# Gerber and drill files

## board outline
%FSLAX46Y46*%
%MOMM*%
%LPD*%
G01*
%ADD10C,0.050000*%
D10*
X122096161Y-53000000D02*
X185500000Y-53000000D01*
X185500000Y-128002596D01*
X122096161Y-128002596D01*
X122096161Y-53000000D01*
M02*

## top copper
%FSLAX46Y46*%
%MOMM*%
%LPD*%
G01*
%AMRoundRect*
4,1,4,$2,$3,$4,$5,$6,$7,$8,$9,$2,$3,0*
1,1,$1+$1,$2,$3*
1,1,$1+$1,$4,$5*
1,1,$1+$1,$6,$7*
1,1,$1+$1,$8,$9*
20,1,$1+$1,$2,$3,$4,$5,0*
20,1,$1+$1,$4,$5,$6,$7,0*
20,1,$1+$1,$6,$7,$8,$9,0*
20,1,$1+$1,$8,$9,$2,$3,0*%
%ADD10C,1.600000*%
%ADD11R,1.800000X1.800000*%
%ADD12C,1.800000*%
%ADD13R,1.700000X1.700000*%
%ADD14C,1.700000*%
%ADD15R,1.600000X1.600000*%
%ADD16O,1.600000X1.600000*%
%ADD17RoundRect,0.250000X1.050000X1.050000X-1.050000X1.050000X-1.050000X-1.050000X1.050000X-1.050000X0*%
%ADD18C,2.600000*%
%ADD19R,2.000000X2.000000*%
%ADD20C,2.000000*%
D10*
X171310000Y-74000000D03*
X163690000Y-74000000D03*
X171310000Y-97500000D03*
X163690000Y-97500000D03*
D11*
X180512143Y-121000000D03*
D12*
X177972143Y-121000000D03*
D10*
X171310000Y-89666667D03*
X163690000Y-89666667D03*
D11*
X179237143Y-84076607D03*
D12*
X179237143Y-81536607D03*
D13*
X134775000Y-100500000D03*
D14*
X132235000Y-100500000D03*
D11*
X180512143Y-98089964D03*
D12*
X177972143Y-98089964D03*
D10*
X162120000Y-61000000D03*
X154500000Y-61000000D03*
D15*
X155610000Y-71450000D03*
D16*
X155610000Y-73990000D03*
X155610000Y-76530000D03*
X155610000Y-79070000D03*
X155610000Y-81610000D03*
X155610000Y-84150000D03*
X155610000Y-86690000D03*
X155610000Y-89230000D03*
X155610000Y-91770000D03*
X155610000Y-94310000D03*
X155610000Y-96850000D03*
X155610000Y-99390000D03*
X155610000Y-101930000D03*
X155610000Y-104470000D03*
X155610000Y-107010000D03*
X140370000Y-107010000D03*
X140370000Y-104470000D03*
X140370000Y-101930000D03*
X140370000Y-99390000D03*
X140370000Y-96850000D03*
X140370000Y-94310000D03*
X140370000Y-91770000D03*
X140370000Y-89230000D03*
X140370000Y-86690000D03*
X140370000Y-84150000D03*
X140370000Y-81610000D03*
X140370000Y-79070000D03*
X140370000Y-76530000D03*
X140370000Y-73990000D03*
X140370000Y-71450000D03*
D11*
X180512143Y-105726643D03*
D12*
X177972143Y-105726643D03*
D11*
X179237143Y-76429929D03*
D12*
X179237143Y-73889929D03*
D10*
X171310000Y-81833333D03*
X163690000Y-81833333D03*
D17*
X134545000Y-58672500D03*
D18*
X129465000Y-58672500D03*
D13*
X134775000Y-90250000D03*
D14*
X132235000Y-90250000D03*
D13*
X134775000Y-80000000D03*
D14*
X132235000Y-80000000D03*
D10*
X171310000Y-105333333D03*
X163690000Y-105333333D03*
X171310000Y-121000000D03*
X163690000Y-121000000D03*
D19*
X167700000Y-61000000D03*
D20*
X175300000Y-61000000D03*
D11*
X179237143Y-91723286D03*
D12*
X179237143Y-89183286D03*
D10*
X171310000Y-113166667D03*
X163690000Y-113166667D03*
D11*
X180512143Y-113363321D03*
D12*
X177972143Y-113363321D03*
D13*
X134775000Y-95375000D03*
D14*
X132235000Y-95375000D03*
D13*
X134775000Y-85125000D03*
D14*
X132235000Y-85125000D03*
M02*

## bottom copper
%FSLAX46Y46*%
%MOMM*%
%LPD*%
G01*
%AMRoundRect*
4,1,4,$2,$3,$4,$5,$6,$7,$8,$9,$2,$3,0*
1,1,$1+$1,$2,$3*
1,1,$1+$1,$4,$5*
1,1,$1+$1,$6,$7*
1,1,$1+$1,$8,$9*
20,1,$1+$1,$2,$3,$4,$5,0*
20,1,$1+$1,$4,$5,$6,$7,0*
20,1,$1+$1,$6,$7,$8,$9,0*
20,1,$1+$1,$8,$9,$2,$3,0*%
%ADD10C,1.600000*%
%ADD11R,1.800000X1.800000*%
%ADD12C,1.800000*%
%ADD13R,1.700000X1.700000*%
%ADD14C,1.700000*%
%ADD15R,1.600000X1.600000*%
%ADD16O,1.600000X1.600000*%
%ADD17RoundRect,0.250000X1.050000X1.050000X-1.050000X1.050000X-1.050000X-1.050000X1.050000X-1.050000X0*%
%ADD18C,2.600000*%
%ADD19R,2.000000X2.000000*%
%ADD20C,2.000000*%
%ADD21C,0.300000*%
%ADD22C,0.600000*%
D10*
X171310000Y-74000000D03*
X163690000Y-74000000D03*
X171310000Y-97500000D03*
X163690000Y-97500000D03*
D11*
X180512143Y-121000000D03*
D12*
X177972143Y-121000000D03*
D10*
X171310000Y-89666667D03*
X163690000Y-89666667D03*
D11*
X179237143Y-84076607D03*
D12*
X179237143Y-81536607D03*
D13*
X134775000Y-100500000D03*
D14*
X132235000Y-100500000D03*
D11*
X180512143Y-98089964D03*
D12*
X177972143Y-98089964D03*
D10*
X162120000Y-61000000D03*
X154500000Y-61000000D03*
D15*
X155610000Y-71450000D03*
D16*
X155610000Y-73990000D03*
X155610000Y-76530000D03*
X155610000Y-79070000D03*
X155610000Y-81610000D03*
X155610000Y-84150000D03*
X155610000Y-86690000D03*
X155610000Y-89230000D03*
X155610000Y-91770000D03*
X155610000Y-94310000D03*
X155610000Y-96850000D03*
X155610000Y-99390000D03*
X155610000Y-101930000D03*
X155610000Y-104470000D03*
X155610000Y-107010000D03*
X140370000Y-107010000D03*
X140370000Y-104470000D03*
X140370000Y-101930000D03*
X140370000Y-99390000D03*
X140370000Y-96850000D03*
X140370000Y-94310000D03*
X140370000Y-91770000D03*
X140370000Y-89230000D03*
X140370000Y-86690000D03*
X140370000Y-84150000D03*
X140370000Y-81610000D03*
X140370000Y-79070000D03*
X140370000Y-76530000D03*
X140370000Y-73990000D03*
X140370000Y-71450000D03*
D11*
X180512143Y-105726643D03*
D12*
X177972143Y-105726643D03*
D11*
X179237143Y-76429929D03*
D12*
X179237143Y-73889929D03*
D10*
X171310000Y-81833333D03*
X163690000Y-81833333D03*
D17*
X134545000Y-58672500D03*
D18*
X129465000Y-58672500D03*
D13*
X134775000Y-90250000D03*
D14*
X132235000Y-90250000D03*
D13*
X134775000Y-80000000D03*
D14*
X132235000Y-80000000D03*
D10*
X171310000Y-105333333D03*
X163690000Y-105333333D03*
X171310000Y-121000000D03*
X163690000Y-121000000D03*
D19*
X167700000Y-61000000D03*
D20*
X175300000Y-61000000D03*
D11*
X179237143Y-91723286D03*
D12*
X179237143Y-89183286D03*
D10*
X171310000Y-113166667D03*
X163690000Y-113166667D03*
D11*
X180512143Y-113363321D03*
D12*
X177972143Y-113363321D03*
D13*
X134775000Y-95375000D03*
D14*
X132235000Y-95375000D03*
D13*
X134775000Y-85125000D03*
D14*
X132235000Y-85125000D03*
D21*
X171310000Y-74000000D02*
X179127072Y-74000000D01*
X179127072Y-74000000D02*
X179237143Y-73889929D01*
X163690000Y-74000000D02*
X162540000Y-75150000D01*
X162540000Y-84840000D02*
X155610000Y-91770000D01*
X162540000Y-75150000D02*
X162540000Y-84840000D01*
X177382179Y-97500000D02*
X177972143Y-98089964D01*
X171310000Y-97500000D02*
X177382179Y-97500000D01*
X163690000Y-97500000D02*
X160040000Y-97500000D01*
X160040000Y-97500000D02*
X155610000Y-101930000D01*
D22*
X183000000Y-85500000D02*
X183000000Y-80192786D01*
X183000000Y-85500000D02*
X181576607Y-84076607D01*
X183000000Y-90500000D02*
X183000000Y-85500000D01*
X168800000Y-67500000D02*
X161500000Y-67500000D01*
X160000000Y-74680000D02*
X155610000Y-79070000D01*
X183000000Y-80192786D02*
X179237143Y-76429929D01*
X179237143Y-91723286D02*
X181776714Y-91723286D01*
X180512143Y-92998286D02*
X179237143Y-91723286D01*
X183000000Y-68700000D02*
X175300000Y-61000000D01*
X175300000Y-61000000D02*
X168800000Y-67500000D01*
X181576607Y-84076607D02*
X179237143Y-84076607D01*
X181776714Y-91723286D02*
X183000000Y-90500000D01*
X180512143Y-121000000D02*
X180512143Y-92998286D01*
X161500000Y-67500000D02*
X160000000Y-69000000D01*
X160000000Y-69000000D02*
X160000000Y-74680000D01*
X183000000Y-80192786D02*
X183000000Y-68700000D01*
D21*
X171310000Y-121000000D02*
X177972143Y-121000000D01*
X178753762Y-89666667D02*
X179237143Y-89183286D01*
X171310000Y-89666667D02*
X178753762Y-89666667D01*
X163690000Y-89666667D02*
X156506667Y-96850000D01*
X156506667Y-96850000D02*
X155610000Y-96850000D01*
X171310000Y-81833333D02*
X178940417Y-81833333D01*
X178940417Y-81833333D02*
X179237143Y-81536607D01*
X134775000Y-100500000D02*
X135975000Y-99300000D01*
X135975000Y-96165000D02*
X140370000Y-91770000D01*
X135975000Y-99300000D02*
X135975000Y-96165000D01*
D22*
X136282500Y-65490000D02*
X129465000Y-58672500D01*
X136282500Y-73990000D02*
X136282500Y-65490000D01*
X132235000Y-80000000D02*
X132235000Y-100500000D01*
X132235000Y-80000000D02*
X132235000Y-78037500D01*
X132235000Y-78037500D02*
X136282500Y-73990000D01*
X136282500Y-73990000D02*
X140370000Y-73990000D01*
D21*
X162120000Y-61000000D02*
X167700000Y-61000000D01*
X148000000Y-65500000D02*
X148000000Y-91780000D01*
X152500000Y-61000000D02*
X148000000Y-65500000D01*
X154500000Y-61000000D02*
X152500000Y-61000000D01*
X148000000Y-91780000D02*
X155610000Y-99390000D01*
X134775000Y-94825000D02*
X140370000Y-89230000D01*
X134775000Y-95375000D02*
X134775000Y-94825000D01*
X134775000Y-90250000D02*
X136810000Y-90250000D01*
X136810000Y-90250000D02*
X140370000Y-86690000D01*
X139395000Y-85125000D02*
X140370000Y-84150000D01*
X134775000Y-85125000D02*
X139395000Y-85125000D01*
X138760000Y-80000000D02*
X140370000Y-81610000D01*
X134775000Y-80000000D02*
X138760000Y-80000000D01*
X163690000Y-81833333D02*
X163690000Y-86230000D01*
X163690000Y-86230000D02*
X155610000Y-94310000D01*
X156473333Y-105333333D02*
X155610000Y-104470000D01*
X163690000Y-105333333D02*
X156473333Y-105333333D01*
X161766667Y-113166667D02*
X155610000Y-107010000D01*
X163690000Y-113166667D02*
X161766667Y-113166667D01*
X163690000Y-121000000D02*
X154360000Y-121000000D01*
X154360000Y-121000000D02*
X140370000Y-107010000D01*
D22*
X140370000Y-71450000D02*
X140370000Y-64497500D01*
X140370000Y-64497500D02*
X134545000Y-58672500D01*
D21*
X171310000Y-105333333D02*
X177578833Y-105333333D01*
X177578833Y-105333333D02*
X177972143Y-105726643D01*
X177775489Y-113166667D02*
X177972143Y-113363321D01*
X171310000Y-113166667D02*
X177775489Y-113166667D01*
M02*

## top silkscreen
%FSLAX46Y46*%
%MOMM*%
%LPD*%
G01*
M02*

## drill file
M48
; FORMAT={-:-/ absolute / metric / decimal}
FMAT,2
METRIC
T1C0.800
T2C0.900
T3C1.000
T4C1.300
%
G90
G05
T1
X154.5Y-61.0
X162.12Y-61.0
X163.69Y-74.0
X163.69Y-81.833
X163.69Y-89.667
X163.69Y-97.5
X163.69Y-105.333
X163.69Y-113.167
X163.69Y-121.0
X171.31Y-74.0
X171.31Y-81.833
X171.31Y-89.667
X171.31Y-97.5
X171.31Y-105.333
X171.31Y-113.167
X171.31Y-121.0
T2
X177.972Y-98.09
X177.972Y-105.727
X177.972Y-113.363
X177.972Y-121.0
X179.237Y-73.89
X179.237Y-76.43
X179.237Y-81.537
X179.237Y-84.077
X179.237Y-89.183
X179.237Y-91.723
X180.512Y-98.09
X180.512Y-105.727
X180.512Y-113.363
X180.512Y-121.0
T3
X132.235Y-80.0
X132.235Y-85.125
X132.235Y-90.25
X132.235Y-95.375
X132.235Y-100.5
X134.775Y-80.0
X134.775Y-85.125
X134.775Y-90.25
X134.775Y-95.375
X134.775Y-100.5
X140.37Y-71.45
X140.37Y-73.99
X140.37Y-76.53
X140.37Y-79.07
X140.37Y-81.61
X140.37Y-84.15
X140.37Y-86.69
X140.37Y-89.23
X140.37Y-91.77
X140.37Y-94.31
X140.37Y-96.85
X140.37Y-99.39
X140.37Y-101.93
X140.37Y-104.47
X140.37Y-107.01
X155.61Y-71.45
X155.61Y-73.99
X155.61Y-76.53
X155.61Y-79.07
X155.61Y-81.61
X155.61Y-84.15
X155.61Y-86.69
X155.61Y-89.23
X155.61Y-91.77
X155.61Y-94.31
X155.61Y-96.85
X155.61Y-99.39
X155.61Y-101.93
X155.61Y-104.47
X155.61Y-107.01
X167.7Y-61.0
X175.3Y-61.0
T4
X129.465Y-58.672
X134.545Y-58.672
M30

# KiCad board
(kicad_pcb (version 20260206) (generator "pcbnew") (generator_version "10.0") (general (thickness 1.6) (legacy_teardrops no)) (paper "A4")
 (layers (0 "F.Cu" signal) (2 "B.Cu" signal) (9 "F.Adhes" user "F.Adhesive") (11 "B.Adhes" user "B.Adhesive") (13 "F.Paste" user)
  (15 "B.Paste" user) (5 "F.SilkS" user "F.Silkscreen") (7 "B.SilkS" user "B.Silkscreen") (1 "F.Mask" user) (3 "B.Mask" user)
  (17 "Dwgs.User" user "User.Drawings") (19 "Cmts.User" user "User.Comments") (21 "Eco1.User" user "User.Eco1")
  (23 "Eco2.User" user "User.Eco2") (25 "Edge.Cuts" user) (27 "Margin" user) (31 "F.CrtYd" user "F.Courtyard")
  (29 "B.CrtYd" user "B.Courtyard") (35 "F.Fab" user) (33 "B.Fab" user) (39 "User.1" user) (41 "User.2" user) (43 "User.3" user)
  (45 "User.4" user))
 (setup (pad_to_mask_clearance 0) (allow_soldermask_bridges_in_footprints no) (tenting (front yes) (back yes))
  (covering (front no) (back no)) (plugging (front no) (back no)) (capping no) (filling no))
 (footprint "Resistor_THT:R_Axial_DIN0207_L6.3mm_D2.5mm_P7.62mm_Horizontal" (layer "B.Cu") (at 171.31 74 180)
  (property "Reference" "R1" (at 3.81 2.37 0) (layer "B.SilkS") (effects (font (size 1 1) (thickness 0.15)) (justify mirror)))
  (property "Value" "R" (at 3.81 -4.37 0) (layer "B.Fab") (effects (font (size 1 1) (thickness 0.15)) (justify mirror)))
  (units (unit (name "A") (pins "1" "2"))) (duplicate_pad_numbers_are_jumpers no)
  (pad "1" thru_hole circle (at 0 0 180) (size 1.6 1.6) (drill 0.8) (layers "*.Cu" "*.Mask") (remove_unused_layers no)
   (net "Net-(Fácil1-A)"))
  (pad "2" thru_hole circle (at 7.62 0 180) (size 1.6 1.6) (drill 0.8) (layers "*.Cu" "*.Mask") (remove_unused_layers no)
   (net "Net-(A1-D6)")))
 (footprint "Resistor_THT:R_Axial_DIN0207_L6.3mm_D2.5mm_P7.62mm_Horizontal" (layer "B.Cu") (at 171.31 97.5 180)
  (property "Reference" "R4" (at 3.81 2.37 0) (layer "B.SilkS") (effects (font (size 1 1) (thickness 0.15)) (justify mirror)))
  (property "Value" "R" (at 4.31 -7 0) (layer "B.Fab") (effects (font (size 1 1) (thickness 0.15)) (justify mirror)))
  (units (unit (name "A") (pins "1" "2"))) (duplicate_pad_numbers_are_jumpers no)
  (pad "1" thru_hole circle (at 0 0 180) (size 1.6 1.6) (drill 0.8) (layers "*.Cu" "*.Mask") (remove_unused_layers no)
   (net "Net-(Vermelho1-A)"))
  (pad "2" thru_hole circle (at 7.62 0 180) (size 1.6 1.6) (drill 0.8) (layers "*.Cu" "*.Mask") (remove_unused_layers no)
   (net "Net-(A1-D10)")))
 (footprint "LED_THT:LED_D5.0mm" (layer "B.Cu") (at 180.512143 121 180)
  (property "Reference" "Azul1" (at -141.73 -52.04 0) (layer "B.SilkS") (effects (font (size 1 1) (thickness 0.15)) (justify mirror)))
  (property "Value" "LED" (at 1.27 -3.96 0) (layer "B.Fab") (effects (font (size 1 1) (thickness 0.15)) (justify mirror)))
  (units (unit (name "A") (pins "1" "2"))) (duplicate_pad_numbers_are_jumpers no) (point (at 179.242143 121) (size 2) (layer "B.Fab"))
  (pad "1" thru_hole rect (at 0 0 180) (size 1.8 1.8) (drill 0.9) (layers "*.Cu" "*.Mask") (remove_unused_layers no)
   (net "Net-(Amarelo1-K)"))
  (pad "2" thru_hole circle (at 2.54 0 180) (size 1.8 1.8) (drill 0.9) (layers "*.Cu" "*.Mask") (remove_unused_layers no)
   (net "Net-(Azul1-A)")))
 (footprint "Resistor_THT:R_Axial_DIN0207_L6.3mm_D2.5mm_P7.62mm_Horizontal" (layer "B.Cu") (at 171.31 89.666667 180)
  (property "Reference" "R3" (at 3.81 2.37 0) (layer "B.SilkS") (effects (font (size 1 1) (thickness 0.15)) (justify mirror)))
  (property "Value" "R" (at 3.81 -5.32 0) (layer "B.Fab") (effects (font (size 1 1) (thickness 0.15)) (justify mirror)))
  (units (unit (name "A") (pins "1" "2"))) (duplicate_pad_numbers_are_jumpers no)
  (pad "1" thru_hole circle (at 0 0 180) (size 1.6 1.6) (drill 0.8) (layers "*.Cu" "*.Mask") (remove_unused_layers no)
   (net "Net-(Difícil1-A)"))
  (pad "2" thru_hole circle (at 7.62 0 180) (size 1.6 1.6) (drill 0.8) (layers "*.Cu" "*.Mask") (remove_unused_layers no)
   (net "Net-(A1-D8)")))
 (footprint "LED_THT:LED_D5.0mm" (layer "B.Cu") (at 179.237143 84.076607 90)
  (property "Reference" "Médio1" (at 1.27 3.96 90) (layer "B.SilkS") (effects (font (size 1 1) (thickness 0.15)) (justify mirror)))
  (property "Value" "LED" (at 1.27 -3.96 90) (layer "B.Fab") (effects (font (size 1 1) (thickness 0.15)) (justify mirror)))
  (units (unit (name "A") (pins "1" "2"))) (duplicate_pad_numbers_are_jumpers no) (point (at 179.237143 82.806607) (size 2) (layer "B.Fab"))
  (pad "1" thru_hole rect (at 0 0 90) (size 1.8 1.8) (drill 0.9) (layers "*.Cu" "*.Mask") (remove_unused_layers no) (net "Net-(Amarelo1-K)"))
  (pad "2" thru_hole circle (at 2.54 0 90) (size 1.8 1.8) (drill 0.9) (layers "*.Cu" "*.Mask") (remove_unused_layers no)
   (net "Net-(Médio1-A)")))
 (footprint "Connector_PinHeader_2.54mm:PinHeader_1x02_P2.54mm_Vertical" (layer "B.Cu") (at 134.775 100.5 90)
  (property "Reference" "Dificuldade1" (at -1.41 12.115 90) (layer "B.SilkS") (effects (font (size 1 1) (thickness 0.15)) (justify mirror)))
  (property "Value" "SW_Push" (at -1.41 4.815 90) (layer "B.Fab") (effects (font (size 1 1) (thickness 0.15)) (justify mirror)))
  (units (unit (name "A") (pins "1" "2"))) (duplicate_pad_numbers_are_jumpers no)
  (pad "1" thru_hole rect (at 0 0 90) (size 1.7 1.7) (drill 1) (layers "*.Cu" "*.Mask") (remove_unused_layers no) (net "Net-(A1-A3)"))
  (pad "2" thru_hole circle (at 0 -2.54 90) (size 1.7 1.7) (drill 1) (layers "*.Cu" "*.Mask") (remove_unused_layers no)
   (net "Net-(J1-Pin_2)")))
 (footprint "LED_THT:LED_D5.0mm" (layer "B.Cu") (at 180.512143 98.089964 180)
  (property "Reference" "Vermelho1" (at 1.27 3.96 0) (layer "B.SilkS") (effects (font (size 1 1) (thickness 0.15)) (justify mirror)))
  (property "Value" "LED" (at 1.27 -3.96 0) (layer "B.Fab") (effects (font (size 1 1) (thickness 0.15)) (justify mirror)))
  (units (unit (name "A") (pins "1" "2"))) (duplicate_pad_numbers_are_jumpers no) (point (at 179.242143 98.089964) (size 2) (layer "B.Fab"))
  (pad "1" thru_hole rect (at 0 0 180) (size 1.8 1.8) (drill 0.9) (layers "*.Cu" "*.Mask") (remove_unused_layers no)
   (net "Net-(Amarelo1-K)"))
  (pad "2" thru_hole circle (at 2.54 0 180) (size 1.8 1.8) (drill 0.9) (layers "*.Cu" "*.Mask") (remove_unused_layers no)
   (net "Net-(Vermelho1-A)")))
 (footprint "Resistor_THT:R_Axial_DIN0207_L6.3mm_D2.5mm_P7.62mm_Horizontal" (layer "B.Cu") (at 162.12 61 180)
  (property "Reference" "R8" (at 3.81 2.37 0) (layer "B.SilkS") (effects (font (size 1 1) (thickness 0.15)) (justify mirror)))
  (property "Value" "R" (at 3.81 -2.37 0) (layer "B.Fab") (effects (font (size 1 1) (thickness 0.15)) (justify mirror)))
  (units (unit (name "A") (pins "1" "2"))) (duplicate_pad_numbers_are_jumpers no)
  (pad "1" thru_hole circle (at 0 0 180) (size 1.6 1.6) (drill 0.8) (layers "*.Cu" "*.Mask") (remove_unused_layers no) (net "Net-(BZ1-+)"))
  (pad "2" thru_hole circle (at 7.62 0 180) (size 1.6 1.6) (drill 0.8) (layers "*.Cu" "*.Mask") (remove_unused_layers no)
   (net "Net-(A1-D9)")))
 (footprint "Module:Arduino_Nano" (layer "B.Cu") (at 155.61 71.45 180)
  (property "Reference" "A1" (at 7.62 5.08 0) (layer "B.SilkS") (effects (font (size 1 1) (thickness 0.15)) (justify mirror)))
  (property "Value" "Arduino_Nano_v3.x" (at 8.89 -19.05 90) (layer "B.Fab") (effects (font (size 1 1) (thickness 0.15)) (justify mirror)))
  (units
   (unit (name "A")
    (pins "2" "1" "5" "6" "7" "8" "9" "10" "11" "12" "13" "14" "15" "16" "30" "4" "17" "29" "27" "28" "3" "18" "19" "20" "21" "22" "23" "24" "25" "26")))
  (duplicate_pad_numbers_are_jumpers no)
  (pad "1" thru_hole rect (at 0 0 180) (size 1.6 1.6) (drill 1) (layers "*.Cu" "*.Mask") (remove_unused_layers no)
   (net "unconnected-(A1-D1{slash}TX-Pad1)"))
  (pad "2" thru_hole oval (at 0 -2.54 180) (size 1.6 1.6) (drill 1) (layers "*.Cu" "*.Mask") (remove_unused_layers no)
   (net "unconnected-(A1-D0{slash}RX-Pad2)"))
  (pad "3" thru_hole oval (at 0 -5.08 180) (size 1.6 1.6) (drill 1) (layers "*.Cu" "*.Mask") (remove_unused_layers no)
   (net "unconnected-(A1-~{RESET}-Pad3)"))
  (pad "4" thru_hole oval (at 0 -7.62 180) (size 1.6 1.6) (drill 1) (layers "*.Cu" "*.Mask") (remove_unused_layers no)
   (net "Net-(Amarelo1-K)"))
  (pad "5" thru_hole oval (at 0 -10.16 180) (size 1.6 1.6) (drill 1) (layers "*.Cu" "*.Mask") (remove_unused_layers no) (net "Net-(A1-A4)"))
  (pad "6" thru_hole oval (at 0 -12.7 180) (size 1.6 1.6) (drill 1) (layers "*.Cu" "*.Mask") (remove_unused_layers no) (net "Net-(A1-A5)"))
  (pad "7" thru_hole oval (at 0 -15.24 180) (size 1.6 1.6) (drill 1) (layers "*.Cu" "*.Mask") (remove_unused_layers no) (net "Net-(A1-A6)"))
  (pad "8" thru_hole oval (at 0 -17.78 180) (size 1.6 1.6) (drill 1) (layers "*.Cu" "*.Mask") (remove_unused_layers no) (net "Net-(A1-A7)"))
  (pad "9" thru_hole oval (at 0 -20.32 180) (size 1.6 1.6) (drill 1) (layers "*.Cu" "*.Mask") (remove_unused_layers no) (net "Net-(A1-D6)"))
  (pad "10" thru_hole oval (at 0 -22.86 180) (size 1.6 1.6) (drill 1) (layers "*.Cu" "*.Mask") (remove_unused_layers no) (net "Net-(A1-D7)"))
  (pad "11" thru_hole oval (at 0 -25.4 180) (size 1.6 1.6) (drill 1) (layers "*.Cu" "*.Mask") (remove_unused_layers no) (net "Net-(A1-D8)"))
  (pad "12" thru_hole oval (at 0 -27.94 180) (size 1.6 1.6) (drill 1) (layers "*.Cu" "*.Mask") (remove_unused_layers no) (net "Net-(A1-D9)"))
  (pad "13" thru_hole oval (at 0 -30.48 180) (size 1.6 1.6) (drill 1) (layers "*.Cu" "*.Mask") (remove_unused_layers no)
   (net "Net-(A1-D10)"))
  (pad "14" thru_hole oval (at 0 -33.02 180) (size 1.6 1.6) (drill 1) (layers "*.Cu" "*.Mask") (remove_unused_layers no)
   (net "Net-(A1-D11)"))
  (pad "15" thru_hole oval (at 0 -35.56 180) (size 1.6 1.6) (drill 1) (layers "*.Cu" "*.Mask") (remove_unused_layers no)
   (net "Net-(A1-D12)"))
  (pad "16" thru_hole oval (at 15.24 -35.56 180) (size 1.6 1.6) (drill 1) (layers "*.Cu" "*.Mask") (remove_unused_layers no)
   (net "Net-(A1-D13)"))
  (pad "17" thru_hole oval (at 15.24 -33.02 180) (size 1.6 1.6) (drill 1) (layers "*.Cu" "*.Mask") (remove_unused_layers no)
   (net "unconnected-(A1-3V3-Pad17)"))
  (pad "18" thru_hole oval (at 15.24 -30.48 180) (size 1.6 1.6) (drill 1) (layers "*.Cu" "*.Mask") (remove_unused_layers no)
   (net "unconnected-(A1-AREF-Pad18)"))
  (pad "19" thru_hole oval (at 15.24 -27.94 180) (size 1.6 1.6) (drill 1) (layers "*.Cu" "*.Mask") (remove_unused_layers no)
   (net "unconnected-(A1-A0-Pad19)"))
  (pad "20" thru_hole oval (at 15.24 -25.4 180) (size 1.6 1.6) (drill 1) (layers "*.Cu" "*.Mask") (remove_unused_layers no)
   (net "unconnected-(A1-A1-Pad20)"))
  (pad "21" thru_hole oval (at 15.24 -22.86 180) (size 1.6 1.6) (drill 1) (layers "*.Cu" "*.Mask") (remove_unused_layers no)
   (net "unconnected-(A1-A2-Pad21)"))
  (pad "22" thru_hole oval (at 15.24 -20.32 180) (size 1.6 1.6) (drill 1) (layers "*.Cu" "*.Mask") (remove_unused_layers no)
   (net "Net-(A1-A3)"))
  (pad "23" thru_hole oval (at 15.24 -17.78 180) (size 1.6 1.6) (drill 1) (layers "*.Cu" "*.Mask") (remove_unused_layers no)
   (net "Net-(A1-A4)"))
  (pad "24" thru_hole oval (at 15.24 -15.24 180) (size 1.6 1.6) (drill 1) (layers "*.Cu" "*.Mask") (remove_unused_layers no)
   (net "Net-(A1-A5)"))
  (pad "25" thru_hole oval (at 15.24 -12.7 180) (size 1.6 1.6) (drill 1) (layers "*.Cu" "*.Mask") (remove_unused_layers no)
   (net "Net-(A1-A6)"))
  (pad "26" thru_hole oval (at 15.24 -10.16 180) (size 1.6 1.6) (drill 1) (layers "*.Cu" "*.Mask") (remove_unused_layers no)
   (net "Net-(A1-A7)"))
  (pad "27" thru_hole oval (at 15.24 -7.62 180) (size 1.6 1.6) (drill 1) (layers "*.Cu" "*.Mask") (remove_unused_layers no)
   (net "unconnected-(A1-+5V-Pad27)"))
  (pad "28" thru_hole oval (at 15.24 -5.08 180) (size 1.6 1.6) (drill 1) (layers "*.Cu" "*.Mask") (remove_unused_layers no)
   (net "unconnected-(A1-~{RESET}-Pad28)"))
  (pad "29" thru_hole oval (at 15.24 -2.54 180) (size 1.6 1.6) (drill 1) (layers "*.Cu" "*.Mask") (remove_unused_layers no)
   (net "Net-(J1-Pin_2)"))
  (pad "30" thru_hole oval (at 15.24 0 180) (size 1.6 1.6) (drill 1) (layers "*.Cu" "*.Mask") (remove_unused_layers no) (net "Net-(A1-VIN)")))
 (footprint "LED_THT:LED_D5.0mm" (layer "B.Cu") (at 180.512143 105.726643 180)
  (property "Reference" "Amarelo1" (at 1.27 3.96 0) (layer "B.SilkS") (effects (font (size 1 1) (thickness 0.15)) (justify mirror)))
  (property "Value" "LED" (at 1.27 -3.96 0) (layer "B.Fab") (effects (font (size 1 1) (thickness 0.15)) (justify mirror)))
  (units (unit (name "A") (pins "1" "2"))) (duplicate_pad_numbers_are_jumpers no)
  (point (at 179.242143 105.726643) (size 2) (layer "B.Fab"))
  (pad "1" thru_hole rect (at 0 0 180) (size 1.8 1.8) (drill 0.9) (layers "*.Cu" "*.Mask") (remove_unused_layers no)
   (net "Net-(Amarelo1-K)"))
  (pad "2" thru_hole circle (at 2.54 0 180) (size 1.8 1.8) (drill 0.9) (layers "*.Cu" "*.Mask") (remove_unused_layers no)
   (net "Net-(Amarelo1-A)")))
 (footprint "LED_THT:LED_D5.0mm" (layer "B.Cu") (at 179.237143 76.429929 90)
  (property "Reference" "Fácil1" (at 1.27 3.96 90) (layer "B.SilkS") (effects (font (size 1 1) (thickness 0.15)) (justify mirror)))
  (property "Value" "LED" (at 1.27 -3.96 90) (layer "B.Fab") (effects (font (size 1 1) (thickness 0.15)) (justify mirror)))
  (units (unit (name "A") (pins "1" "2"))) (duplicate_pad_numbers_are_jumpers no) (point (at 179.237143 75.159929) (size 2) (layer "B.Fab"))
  (pad "1" thru_hole rect (at 0 0 90) (size 1.8 1.8) (drill 0.9) (layers "*.Cu" "*.Mask") (remove_unused_layers no) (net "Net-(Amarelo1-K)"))
  (pad "2" thru_hole circle (at 2.54 0 90) (size 1.8 1.8) (drill 0.9) (layers "*.Cu" "*.Mask") (remove_unused_layers no)
   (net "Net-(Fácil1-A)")))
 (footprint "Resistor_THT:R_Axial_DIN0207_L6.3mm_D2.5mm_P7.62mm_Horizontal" (layer "B.Cu") (at 171.31 81.833333 180)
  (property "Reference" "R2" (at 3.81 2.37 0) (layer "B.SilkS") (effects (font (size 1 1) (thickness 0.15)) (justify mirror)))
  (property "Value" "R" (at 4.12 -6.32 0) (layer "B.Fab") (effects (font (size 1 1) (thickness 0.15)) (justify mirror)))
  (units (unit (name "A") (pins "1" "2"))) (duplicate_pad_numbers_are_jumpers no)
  (pad "1" thru_hole circle (at 0 0 180) (size 1.6 1.6) (drill 0.8) (layers "*.Cu" "*.Mask") (remove_unused_layers no)
   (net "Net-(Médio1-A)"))
  (pad "2" thru_hole circle (at 7.62 0 180) (size 1.6 1.6) (drill 0.8) (layers "*.Cu" "*.Mask") (remove_unused_layers no)
   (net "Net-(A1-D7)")))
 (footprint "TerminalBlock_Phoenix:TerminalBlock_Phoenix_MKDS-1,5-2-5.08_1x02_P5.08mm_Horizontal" (layer "B.Cu") (at 134.545 58.6725 180)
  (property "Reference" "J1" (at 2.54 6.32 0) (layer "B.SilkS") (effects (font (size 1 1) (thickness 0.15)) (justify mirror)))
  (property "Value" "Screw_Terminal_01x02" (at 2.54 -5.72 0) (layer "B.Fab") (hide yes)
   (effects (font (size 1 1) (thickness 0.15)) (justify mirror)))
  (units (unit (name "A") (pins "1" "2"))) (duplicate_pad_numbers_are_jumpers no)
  (pad "1" thru_hole roundrect (at 0 0 180) (size 2.6 2.6) (drill 1.3) (layers "*.Cu" "*.Mask") (remove_unused_layers no)
   (roundrect_rratio 0.096154) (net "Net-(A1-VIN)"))
  (pad "2" thru_hole circle (at 5.08 0 180) (size 2.6 2.6) (drill 1.3) (layers "*.Cu" "*.Mask") (remove_unused_layers no)
   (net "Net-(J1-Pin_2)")))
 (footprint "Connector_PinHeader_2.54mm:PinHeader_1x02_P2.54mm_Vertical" (layer "B.Cu") (at 134.775 90.25 90)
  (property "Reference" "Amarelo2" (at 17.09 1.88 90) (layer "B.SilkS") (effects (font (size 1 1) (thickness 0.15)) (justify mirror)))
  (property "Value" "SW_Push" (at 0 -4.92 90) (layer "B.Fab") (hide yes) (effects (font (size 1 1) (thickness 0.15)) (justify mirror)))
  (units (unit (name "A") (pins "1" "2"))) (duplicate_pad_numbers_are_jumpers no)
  (pad "1" thru_hole rect (at 0 0 90) (size 1.7 1.7) (drill 1) (layers "*.Cu" "*.Mask") (remove_unused_layers no) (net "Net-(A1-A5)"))
  (pad "2" thru_hole circle (at 0 -2.54 90) (size 1.7 1.7) (drill 1) (layers "*.Cu" "*.Mask") (remove_unused_layers no)
   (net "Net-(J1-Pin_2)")))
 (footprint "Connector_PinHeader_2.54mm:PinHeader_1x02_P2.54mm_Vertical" (layer "B.Cu") (at 134.775 80 90)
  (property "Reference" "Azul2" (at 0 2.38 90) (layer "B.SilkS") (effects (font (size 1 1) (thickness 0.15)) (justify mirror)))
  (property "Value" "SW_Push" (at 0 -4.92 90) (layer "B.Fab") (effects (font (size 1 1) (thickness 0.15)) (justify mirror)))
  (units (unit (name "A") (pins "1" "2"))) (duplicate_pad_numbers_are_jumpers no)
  (pad "1" thru_hole rect (at 0 0 90) (size 1.7 1.7) (drill 1) (layers "*.Cu" "*.Mask") (remove_unused_layers no) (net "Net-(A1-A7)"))
  (pad "2" thru_hole circle (at 0 -2.54 90) (size 1.7 1.7) (drill 1) (layers "*.Cu" "*.Mask") (remove_unused_layers no)
   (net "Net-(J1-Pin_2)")))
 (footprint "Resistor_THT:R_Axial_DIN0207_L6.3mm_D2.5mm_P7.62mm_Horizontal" (layer "B.Cu") (at 171.31 105.333333 180)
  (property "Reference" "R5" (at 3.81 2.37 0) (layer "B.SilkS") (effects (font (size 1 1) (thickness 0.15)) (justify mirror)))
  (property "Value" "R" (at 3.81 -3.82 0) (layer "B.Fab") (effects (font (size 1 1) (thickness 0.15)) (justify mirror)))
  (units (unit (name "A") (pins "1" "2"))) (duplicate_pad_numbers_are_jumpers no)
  (pad "1" thru_hole circle (at 0 0 180) (size 1.6 1.6) (drill 0.8) (layers "*.Cu" "*.Mask") (remove_unused_layers no)
   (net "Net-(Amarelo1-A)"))
  (pad "2" thru_hole circle (at 7.62 0 180) (size 1.6 1.6) (drill 0.8) (layers "*.Cu" "*.Mask") (remove_unused_layers no)
   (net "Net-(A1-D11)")))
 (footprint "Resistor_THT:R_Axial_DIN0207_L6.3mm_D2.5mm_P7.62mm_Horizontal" (layer "B.Cu") (at 171.31 121 180)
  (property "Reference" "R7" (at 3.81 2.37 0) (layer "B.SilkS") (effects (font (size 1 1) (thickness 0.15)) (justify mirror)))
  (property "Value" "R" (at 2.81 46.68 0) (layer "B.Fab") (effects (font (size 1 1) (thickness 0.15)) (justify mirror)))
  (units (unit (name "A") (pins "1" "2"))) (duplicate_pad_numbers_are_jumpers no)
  (pad "1" thru_hole circle (at 0 0 180) (size 1.6 1.6) (drill 0.8) (layers "*.Cu" "*.Mask") (remove_unused_layers no) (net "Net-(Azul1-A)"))
  (pad "2" thru_hole circle (at 7.62 0 180) (size 1.6 1.6) (drill 0.8) (layers "*.Cu" "*.Mask") (remove_unused_layers no)
   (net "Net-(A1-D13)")))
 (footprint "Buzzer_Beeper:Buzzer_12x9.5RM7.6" (layer "B.Cu") (at 167.7 61)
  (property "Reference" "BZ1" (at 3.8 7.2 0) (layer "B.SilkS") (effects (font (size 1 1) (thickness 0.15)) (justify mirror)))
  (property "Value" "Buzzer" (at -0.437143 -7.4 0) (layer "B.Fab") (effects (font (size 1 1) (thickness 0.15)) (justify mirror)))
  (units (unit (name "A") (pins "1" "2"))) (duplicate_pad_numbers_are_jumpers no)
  (pad "1" thru_hole rect (at 0 0) (size 2 2) (drill 1) (layers "*.Cu" "*.Mask") (remove_unused_layers no) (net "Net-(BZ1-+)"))
  (pad "2" thru_hole circle (at 7.6 0) (size 2 2) (drill 1) (layers "*.Cu" "*.Mask") (remove_unused_layers no) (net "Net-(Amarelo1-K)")))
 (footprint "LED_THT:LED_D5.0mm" (layer "B.Cu") (at 179.237143 91.723286 90)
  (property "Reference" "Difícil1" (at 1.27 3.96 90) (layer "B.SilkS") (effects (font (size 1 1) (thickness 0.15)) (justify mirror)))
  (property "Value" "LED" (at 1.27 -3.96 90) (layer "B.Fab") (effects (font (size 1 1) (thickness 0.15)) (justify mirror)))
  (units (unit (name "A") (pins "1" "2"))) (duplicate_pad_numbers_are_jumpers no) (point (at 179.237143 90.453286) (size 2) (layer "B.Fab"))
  (pad "1" thru_hole rect (at 0 0 90) (size 1.8 1.8) (drill 0.9) (layers "*.Cu" "*.Mask") (remove_unused_layers no) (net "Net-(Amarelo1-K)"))
  (pad "2" thru_hole circle (at 2.54 0 90) (size 1.8 1.8) (drill 0.9) (layers "*.Cu" "*.Mask") (remove_unused_layers no)
   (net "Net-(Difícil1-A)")))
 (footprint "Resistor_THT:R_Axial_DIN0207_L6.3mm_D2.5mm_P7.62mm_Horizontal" (layer "B.Cu") (at 171.31 113.166667 180)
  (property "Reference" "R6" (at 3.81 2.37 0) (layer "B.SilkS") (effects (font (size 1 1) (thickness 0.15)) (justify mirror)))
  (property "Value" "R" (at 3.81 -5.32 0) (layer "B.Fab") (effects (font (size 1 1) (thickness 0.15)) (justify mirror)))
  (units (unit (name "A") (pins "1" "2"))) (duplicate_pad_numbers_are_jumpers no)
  (pad "1" thru_hole circle (at 0 0 180) (size 1.6 1.6) (drill 0.8) (layers "*.Cu" "*.Mask") (remove_unused_layers no)
   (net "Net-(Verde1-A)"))
  (pad "2" thru_hole circle (at 7.62 0 180) (size 1.6 1.6) (drill 0.8) (layers "*.Cu" "*.Mask") (remove_unused_layers no)
   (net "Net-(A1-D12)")))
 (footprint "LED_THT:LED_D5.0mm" (layer "B.Cu") (at 180.512143 113.363321 180)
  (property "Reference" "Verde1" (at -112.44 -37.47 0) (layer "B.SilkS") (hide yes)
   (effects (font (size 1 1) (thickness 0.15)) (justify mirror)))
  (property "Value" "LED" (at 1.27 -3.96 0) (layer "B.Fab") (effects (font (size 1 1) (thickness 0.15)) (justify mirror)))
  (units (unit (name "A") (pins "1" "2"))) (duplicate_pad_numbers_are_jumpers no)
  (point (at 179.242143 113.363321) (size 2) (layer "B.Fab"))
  (pad "1" thru_hole rect (at 0 0 180) (size 1.8 1.8) (drill 0.9) (layers "*.Cu" "*.Mask") (remove_unused_layers no)
   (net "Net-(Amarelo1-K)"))
  (pad "2" thru_hole circle (at 2.54 0 180) (size 1.8 1.8) (drill 0.9) (layers "*.Cu" "*.Mask") (remove_unused_layers no)
   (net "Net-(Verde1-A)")))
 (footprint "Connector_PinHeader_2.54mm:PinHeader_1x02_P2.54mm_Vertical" (layer "B.Cu") (at 134.775 95.375 90)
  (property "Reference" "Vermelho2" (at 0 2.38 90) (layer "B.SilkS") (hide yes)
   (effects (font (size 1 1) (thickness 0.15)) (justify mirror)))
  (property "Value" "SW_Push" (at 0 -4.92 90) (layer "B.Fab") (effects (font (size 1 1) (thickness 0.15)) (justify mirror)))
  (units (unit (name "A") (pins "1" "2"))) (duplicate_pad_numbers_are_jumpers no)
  (pad "1" thru_hole rect (at 0 0 90) (size 1.7 1.7) (drill 1) (layers "*.Cu" "*.Mask") (remove_unused_layers no) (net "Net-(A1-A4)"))
  (pad "2" thru_hole circle (at 0 -2.54 90) (size 1.7 1.7) (drill 1) (layers "*.Cu" "*.Mask") (remove_unused_layers no)
   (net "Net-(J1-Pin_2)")))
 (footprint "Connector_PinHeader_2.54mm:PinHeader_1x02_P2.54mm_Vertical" (layer "B.Cu") (at 134.775 85.125 90)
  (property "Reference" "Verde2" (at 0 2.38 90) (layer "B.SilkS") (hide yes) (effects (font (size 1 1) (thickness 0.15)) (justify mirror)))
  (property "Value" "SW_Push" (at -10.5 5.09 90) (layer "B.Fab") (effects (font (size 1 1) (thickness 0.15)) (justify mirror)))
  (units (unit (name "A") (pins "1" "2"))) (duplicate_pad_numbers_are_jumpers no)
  (pad "1" thru_hole rect (at 0 0 90) (size 1.7 1.7) (drill 1) (layers "*.Cu" "*.Mask") (remove_unused_layers no) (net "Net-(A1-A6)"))
  (pad "2" thru_hole circle (at 0 -2.54 90) (size 1.7 1.7) (drill 1) (layers "*.Cu" "*.Mask") (remove_unused_layers no)
   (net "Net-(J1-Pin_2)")))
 (gr_rect (start 122.096161 53) (end 185.5 128.002596) (stroke (width 0.05) (type default)) (fill no) (layer "Edge.Cuts"))
 (segment (start 171.31 74) (end 179.127072 74) (width 0.3) (layer "B.Cu") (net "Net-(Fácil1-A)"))
 (segment (start 179.127072 74) (end 179.237143 73.889929) (width 0.3) (layer "B.Cu") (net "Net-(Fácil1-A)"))
 (segment (start 163.69 74) (end 162.54 75.15) (width 0.3) (layer "B.Cu") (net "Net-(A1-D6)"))
 (segment (start 162.54 84.84) (end 155.61 91.77) (width 0.3) (layer "B.Cu") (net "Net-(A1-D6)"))
 (segment (start 162.54 75.15) (end 162.54 84.84) (width 0.3) (layer "B.Cu") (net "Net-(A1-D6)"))
 (segment (start 177.382179 97.5) (end 177.972143 98.089964) (width 0.3) (layer "B.Cu") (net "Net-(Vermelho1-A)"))
 (segment (start 171.31 97.5) (end 177.382179 97.5) (width 0.3) (layer "B.Cu") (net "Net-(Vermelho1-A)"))
 (segment (start 163.69 97.5) (end 160.04 97.5) (width 0.3) (layer "B.Cu") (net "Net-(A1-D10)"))
 (segment (start 160.04 97.5) (end 155.61 101.93) (width 0.3) (layer "B.Cu") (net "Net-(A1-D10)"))
 (segment (start 183 85.5) (end 183 80.192786) (width 0.6) (layer "B.Cu") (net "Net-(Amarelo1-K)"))
 (segment (start 183 85.5) (end 181.576607 84.076607) (width 0.6) (layer "B.Cu") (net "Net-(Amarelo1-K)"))
 (segment (start 183 90.5) (end 183 85.5) (width 0.6) (layer "B.Cu") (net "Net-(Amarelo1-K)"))
 (segment (start 168.8 67.5) (end 161.5 67.5) (width 0.6) (layer "B.Cu") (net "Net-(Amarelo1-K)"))
 (segment (start 160 74.68) (end 155.61 79.07) (width 0.6) (layer "B.Cu") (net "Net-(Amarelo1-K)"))
 (segment (start 183 80.192786) (end 179.237143 76.429929) (width 0.6) (layer "B.Cu") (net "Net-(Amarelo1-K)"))
 (segment (start 179.237143 91.723286) (end 181.776714 91.723286) (width 0.6) (layer "B.Cu") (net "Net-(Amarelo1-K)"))
 (segment (start 180.512143 92.998286) (end 179.237143 91.723286) (width 0.6) (layer "B.Cu") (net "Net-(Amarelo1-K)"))
 (segment (start 183 68.7) (end 175.3 61) (width 0.6) (layer "B.Cu") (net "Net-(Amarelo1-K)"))
 (segment (start 175.3 61) (end 168.8 67.5) (width 0.6) (layer "B.Cu") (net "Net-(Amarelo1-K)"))
 (segment (start 181.576607 84.076607) (end 179.237143 84.076607) (width 0.6) (layer "B.Cu") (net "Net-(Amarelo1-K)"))
 (segment (start 181.776714 91.723286) (end 183 90.5) (width 0.6) (layer "B.Cu") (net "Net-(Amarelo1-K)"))
 (segment (start 180.512143 121) (end 180.512143 92.998286) (width 0.6) (layer "B.Cu") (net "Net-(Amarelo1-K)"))
 (segment (start 161.5 67.5) (end 160 69) (width 0.6) (layer "B.Cu") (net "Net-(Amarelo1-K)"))
 (segment (start 160 69) (end 160 74.68) (width 0.6) (layer "B.Cu") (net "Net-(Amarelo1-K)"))
 (segment (start 183 80.192786) (end 183 68.7) (width 0.6) (layer "B.Cu") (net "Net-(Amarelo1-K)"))
 (segment (start 171.31 121) (end 177.972143 121) (width 0.3) (layer "B.Cu") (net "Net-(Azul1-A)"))
 (segment (start 178.753762 89.666667) (end 179.237143 89.183286) (width 0.3) (layer "B.Cu") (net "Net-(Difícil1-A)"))
 (segment (start 171.31 89.666667) (end 178.753762 89.666667) (width 0.3) (layer "B.Cu") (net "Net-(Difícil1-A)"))
 (segment (start 163.69 89.666667) (end 156.506667 96.85) (width 0.3) (layer "B.Cu") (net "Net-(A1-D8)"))
 (segment (start 156.506667 96.85) (end 155.61 96.85) (width 0.3) (layer "B.Cu") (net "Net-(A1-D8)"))
 (segment (start 171.31 81.833333) (end 178.940417 81.833333) (width 0.3) (layer "B.Cu") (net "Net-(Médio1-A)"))
 (segment (start 178.940417 81.833333) (end 179.237143 81.536607) (width 0.3) (layer "B.Cu") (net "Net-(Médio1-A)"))
 (segment (start 134.775 100.5) (end 135.975 99.3) (width 0.3) (layer "B.Cu") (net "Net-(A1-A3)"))
 (segment (start 135.975 96.165) (end 140.37 91.77) (width 0.3) (layer "B.Cu") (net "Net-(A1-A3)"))
 (segment (start 135.975 99.3) (end 135.975 96.165) (width 0.3) (layer "B.Cu") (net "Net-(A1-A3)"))
 (segment (start 136.2825 65.49) (end 129.465 58.6725) (width 0.6) (layer "B.Cu") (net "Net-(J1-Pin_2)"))
 (segment (start 136.2825 73.99) (end 136.2825 65.49) (width 0.6) (layer "B.Cu") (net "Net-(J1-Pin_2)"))
 (segment (start 132.235 80) (end 132.235 100.5) (width 0.6) (layer "B.Cu") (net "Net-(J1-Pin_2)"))
 (segment (start 132.235 80) (end 132.235 78.0375) (width 0.6) (layer "B.Cu") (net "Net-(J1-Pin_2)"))
 (segment (start 132.235 78.0375) (end 136.2825 73.99) (width 0.6) (layer "B.Cu") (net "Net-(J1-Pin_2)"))
 (segment (start 136.2825 73.99) (end 140.37 73.99) (width 0.6) (layer "B.Cu") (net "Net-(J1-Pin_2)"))
 (segment (start 162.12 61) (end 167.7 61) (width 0.3) (layer "B.Cu") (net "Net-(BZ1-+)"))
 (segment (start 148 65.5) (end 148 91.78) (width 0.3) (layer "B.Cu") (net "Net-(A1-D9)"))
 (segment (start 152.5 61) (end 148 65.5) (width 0.3) (layer "B.Cu") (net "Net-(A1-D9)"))
 (segment (start 154.5 61) (end 152.5 61) (width 0.3) (layer "B.Cu") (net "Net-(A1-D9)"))
 (segment (start 148 91.78) (end 155.61 99.39) (width 0.3) (layer "B.Cu") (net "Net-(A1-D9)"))
 (segment (start 134.775 94.825) (end 140.37 89.23) (width 0.3) (layer "B.Cu") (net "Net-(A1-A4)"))
 (segment (start 134.775 95.375) (end 134.775 94.825) (width 0.3) (layer "B.Cu") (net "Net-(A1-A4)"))
 (segment (start 134.775 90.25) (end 136.81 90.25) (width 0.3) (layer "B.Cu") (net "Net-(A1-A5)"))
 (segment (start 136.81 90.25) (end 140.37 86.69) (width 0.3) (layer "B.Cu") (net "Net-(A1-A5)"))
 (segment (start 139.395 85.125) (end 140.37 84.15) (width 0.3) (layer "B.Cu") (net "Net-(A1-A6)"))
 (segment (start 134.775 85.125) (end 139.395 85.125) (width 0.3) (layer "B.Cu") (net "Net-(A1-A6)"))
 (segment (start 138.76 80) (end 140.37 81.61) (width 0.3) (layer "B.Cu") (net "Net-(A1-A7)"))
 (segment (start 134.775 80) (end 138.76 80) (width 0.3) (layer "B.Cu") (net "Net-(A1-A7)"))
 (segment (start 163.69 81.833333) (end 163.69 86.23) (width 0.3) (layer "B.Cu") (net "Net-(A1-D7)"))
 (segment (start 163.69 86.23) (end 155.61 94.31) (width 0.3) (layer "B.Cu") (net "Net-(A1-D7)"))
 (segment (start 156.473333 105.333333) (end 155.61 104.47) (width 0.3) (layer "B.Cu") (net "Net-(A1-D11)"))
 (segment (start 163.69 105.333333) (end 156.473333 105.333333) (width 0.3) (layer "B.Cu") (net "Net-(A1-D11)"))
 (segment (start 161.766667 113.166667) (end 155.61 107.01) (width 0.3) (layer "B.Cu") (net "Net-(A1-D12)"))
 (segment (start 163.69 113.166667) (end 161.766667 113.166667) (width 0.3) (layer "B.Cu") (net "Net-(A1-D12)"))
 (segment (start 163.69 121) (end 154.36 121) (width 0.3) (layer "B.Cu") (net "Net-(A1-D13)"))
 (segment (start 154.36 121) (end 140.37 107.01) (width 0.3) (layer "B.Cu") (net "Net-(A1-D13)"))
 (segment (start 140.37 71.45) (end 140.37 64.4975) (width 0.6) (layer "B.Cu") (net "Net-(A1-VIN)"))
 (segment (start 140.37 64.4975) (end 134.545 58.6725) (width 0.6) (layer "B.Cu") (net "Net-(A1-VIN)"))
 (segment (start 171.31 105.333333) (end 177.578833 105.333333) (width 0.3) (layer "B.Cu") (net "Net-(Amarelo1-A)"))
 (segment (start 177.578833 105.333333) (end 177.972143 105.726643) (width 0.3) (layer "B.Cu") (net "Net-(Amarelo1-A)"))
 (segment (start 177.775489 113.166667) (end 177.972143 113.363321) (width 0.3) (layer "B.Cu") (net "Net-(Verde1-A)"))
 (segment (start 171.31 113.166667) (end 177.775489 113.166667) (width 0.3) (layer "B.Cu") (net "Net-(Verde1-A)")))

